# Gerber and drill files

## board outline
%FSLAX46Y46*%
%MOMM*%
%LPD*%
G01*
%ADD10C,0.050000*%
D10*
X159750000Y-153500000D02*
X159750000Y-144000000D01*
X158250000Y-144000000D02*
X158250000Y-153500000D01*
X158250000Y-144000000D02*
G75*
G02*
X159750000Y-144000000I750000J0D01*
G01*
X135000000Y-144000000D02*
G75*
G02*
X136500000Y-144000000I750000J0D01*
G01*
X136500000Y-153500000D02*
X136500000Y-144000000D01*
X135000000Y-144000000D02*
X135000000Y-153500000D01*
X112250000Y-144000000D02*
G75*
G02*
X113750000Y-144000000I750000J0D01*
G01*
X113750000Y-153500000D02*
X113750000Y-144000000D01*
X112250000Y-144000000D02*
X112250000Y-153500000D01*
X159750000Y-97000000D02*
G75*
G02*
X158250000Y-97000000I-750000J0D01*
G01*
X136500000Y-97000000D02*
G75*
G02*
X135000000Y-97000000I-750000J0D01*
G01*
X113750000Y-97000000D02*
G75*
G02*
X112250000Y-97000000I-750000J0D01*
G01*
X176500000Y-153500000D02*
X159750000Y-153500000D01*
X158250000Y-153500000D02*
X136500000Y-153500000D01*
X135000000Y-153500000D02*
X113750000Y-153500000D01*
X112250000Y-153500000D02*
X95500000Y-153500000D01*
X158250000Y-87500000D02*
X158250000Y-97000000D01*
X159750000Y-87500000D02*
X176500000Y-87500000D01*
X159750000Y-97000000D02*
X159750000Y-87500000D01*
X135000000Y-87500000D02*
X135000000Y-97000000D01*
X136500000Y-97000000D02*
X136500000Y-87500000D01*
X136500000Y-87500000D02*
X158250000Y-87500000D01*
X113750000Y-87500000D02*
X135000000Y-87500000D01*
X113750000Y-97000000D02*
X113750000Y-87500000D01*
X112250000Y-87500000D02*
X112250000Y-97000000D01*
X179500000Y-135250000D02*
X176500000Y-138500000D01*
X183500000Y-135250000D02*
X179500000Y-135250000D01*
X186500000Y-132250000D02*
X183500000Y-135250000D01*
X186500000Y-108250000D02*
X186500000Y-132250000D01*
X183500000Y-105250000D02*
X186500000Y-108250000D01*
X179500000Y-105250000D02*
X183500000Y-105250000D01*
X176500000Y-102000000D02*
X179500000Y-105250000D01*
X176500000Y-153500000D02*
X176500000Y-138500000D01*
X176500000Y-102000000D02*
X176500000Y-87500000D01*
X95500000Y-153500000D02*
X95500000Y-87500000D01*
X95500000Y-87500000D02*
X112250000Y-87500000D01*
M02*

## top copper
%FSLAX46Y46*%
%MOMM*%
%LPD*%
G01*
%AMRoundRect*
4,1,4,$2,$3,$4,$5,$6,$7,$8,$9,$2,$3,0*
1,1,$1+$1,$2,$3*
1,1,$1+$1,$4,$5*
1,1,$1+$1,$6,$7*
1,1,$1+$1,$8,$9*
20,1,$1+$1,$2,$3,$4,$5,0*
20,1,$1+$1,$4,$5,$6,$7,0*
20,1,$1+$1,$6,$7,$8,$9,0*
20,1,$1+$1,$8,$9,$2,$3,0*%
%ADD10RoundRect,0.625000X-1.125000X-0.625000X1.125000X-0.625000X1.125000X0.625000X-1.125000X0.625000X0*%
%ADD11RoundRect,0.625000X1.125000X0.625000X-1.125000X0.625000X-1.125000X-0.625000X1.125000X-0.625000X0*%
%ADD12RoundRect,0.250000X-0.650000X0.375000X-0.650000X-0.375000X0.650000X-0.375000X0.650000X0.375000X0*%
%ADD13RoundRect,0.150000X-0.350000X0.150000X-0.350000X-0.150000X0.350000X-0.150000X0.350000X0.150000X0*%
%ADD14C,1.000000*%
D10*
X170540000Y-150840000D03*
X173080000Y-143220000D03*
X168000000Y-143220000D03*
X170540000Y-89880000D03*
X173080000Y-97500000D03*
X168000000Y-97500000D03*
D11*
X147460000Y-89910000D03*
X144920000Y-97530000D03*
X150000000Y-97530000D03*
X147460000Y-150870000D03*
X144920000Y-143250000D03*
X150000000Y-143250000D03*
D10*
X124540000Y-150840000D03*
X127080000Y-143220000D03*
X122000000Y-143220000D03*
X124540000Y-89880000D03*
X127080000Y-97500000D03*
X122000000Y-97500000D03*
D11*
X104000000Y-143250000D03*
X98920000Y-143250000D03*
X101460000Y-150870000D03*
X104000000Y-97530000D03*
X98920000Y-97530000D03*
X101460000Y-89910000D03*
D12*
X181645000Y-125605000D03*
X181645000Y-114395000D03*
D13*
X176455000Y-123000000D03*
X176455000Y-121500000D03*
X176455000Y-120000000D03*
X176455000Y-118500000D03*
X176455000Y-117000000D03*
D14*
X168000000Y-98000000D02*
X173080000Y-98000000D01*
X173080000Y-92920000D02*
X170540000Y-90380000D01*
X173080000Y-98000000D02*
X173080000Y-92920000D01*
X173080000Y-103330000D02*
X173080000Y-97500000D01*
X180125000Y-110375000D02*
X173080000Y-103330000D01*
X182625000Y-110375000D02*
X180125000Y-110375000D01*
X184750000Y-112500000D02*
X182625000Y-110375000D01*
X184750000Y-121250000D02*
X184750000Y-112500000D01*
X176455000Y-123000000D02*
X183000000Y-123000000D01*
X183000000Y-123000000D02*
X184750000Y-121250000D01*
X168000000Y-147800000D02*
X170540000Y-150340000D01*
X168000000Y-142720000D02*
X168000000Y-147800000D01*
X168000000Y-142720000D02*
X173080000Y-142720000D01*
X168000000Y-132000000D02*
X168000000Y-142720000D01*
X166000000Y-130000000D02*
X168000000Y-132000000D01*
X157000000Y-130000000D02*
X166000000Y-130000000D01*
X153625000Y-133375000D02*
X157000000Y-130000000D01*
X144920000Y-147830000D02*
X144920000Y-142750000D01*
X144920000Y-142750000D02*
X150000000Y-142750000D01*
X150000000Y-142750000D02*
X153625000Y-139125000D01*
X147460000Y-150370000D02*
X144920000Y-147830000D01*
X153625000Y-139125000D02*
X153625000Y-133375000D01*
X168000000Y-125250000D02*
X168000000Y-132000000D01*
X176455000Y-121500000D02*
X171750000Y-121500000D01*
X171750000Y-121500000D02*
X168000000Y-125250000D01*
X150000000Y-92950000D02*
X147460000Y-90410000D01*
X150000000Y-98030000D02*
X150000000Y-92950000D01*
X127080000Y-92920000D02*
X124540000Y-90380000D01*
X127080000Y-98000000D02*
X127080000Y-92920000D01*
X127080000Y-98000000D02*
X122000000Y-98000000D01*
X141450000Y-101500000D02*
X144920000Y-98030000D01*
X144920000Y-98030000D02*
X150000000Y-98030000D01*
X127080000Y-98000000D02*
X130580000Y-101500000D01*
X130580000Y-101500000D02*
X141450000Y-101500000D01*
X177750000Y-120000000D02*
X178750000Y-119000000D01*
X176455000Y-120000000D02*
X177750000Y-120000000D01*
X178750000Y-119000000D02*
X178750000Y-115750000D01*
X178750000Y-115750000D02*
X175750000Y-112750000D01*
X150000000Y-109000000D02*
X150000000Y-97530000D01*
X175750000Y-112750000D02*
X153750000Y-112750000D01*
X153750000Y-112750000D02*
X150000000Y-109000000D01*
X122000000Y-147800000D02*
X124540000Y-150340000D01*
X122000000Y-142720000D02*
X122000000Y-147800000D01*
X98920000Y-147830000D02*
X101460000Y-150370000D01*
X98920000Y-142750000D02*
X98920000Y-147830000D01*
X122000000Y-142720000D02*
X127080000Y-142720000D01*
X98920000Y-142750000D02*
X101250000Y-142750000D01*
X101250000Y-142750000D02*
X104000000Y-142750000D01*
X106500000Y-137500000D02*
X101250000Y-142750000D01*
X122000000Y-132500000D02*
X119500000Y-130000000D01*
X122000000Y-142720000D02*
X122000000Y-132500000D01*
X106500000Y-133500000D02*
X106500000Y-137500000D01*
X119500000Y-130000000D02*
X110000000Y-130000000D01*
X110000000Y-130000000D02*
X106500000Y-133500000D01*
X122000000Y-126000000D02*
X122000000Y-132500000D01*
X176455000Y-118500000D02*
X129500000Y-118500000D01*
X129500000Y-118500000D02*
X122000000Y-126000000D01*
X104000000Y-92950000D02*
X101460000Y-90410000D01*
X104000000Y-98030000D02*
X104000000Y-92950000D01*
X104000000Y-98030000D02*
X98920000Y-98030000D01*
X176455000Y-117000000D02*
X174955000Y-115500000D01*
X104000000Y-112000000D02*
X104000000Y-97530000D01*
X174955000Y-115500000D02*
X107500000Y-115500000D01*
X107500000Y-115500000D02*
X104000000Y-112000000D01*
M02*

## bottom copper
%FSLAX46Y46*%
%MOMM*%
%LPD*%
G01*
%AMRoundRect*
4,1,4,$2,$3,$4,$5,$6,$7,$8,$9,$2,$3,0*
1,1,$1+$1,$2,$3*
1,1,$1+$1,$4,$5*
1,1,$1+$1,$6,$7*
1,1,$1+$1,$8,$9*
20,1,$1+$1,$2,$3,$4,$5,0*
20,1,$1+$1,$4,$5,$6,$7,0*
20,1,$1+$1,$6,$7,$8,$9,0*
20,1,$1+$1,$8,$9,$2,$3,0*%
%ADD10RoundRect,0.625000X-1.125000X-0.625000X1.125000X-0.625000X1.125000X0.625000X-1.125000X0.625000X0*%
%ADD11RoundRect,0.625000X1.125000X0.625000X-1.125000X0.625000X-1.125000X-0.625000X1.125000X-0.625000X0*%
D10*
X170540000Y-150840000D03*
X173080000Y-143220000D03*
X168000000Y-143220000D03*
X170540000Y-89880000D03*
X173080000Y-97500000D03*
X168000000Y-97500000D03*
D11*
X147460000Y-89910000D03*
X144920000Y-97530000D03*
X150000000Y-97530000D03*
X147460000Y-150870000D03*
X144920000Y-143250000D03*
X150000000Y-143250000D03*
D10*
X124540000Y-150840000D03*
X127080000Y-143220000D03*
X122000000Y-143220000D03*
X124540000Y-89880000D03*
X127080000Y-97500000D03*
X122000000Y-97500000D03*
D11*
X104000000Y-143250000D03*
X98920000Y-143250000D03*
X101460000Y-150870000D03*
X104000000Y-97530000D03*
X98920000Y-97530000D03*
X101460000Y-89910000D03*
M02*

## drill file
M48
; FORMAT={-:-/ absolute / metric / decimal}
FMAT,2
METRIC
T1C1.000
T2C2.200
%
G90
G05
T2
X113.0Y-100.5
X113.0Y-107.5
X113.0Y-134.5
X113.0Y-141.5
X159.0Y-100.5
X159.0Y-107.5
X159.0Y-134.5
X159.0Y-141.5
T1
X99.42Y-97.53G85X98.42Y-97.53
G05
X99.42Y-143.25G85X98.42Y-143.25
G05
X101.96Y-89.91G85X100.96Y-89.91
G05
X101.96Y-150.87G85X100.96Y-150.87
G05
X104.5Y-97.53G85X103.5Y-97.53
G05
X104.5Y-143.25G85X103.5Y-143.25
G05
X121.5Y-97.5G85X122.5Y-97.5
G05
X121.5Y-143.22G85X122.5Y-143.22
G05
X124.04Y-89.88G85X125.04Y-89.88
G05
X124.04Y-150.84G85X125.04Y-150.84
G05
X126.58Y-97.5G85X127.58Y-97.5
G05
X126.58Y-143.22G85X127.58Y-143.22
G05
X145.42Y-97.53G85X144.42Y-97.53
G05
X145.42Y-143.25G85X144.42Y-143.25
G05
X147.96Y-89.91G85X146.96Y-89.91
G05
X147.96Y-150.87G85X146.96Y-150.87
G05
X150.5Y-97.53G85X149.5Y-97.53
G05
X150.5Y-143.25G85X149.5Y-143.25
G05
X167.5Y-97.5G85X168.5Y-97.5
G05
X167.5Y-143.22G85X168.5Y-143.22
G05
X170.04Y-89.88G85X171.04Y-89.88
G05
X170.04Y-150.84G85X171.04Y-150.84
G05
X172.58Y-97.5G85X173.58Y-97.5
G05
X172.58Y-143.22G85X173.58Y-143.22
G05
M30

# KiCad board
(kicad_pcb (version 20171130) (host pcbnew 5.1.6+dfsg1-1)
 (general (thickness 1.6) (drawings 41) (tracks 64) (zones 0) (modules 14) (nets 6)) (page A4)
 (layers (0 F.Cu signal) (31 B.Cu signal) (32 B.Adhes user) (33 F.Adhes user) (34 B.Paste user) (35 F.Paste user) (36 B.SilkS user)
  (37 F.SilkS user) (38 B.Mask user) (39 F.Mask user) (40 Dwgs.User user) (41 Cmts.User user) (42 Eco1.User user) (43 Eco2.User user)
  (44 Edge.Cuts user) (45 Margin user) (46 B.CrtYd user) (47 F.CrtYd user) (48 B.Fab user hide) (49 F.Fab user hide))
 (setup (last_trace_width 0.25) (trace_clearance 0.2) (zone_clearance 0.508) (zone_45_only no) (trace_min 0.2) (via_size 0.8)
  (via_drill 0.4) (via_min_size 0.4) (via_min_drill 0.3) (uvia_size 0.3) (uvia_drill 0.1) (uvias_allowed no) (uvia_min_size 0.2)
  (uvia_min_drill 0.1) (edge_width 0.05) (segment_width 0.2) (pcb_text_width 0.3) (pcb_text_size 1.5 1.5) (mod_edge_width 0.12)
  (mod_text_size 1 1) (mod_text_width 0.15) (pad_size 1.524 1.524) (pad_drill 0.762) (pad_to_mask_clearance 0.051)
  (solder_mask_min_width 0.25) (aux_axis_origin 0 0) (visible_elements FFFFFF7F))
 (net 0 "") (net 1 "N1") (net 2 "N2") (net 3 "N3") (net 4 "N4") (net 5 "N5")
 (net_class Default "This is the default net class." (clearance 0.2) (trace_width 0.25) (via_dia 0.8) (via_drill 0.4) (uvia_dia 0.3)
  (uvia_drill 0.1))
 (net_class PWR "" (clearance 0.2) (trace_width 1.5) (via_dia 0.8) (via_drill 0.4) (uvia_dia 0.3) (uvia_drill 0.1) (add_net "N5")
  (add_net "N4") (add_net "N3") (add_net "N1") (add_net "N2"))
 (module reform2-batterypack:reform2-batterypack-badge (layer F.Cu) (at 136 120.5 90)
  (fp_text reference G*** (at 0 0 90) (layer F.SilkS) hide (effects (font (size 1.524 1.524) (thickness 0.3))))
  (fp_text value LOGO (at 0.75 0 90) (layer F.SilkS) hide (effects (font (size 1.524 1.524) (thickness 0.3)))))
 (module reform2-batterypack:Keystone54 (layer F.Cu) (at 168 98)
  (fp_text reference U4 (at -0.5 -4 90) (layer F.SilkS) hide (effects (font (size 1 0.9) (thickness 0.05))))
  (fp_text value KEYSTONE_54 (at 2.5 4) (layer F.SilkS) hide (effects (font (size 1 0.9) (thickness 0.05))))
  (pad 6 thru_hole roundrect (at 2.54 52.84) (size 3.5 2.5) (drill oval 2 1) (layers *.Cu *.Mask) (roundrect_rratio 0.25) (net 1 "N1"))
  (pad 5 thru_hole roundrect (at 5.08 45.22) (size 3.5 2.5) (drill oval 2 1) (layers *.Cu *.Mask) (roundrect_rratio 0.25) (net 1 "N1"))
  (pad 4 thru_hole roundrect (at 0 45.22) (size 3.5 2.5) (drill oval 2 1) (layers *.Cu *.Mask) (roundrect_rratio 0.25) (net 1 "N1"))
  (pad 3 thru_hole roundrect (at 2.54 -8.12) (size 3.5 2.5) (drill oval 2 1) (layers *.Cu *.Mask) (roundrect_rratio 0.25) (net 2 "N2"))
  (pad 2 thru_hole roundrect (at 5.08 -0.5) (size 3.5 2.5) (drill oval 2 1) (layers *.Cu *.Mask) (roundrect_rratio 0.25) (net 2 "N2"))
  (pad 1 thru_hole roundrect (at 0 -0.5) (size 3.5 2.5) (drill oval 2 1) (layers *.Cu *.Mask) (roundrect_rratio 0.25) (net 2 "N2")))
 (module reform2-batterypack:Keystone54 (layer F.Cu) (at 150 142.75 180)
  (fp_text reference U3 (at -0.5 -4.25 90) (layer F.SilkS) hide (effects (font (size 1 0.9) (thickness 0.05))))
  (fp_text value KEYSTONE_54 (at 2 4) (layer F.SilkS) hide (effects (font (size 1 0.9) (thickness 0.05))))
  (pad 6 thru_hole roundrect (at 2.54 52.84 180) (size 3.5 2.5) (drill oval 2 1) (layers *.Cu *.Mask) (roundrect_rratio 0.25) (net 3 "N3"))
  (pad 5 thru_hole roundrect (at 5.08 45.22 180) (size 3.5 2.5) (drill oval 2 1) (layers *.Cu *.Mask) (roundrect_rratio 0.25) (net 3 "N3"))
  (pad 4 thru_hole roundrect (at 0 45.22 180) (size 3.5 2.5) (drill oval 2 1) (layers *.Cu *.Mask) (roundrect_rratio 0.25) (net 3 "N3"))
  (pad 3 thru_hole roundrect (at 2.54 -8.12 180) (size 3.5 2.5) (drill oval 2 1) (layers *.Cu *.Mask) (roundrect_rratio 0.25) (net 1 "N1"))
  (pad 2 thru_hole roundrect (at 5.08 -0.5 180) (size 3.5 2.5) (drill oval 2 1) (layers *.Cu *.Mask) (roundrect_rratio 0.25) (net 1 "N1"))
  (pad 1 thru_hole roundrect (at 0 -0.5 180) (size 3.5 2.5) (drill oval 2 1) (layers *.Cu *.Mask) (roundrect_rratio 0.25) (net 1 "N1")))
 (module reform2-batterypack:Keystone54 (layer F.Cu) (at 122 98)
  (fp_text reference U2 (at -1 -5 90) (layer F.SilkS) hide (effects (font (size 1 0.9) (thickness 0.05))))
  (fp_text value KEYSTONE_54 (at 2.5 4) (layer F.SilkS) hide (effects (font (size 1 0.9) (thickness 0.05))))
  (pad 6 thru_hole roundrect (at 2.54 52.84) (size 3.5 2.5) (drill oval 2 1) (layers *.Cu *.Mask) (roundrect_rratio 0.25) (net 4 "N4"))
  (pad 5 thru_hole roundrect (at 5.08 45.22) (size 3.5 2.5) (drill oval 2 1) (layers *.Cu *.Mask) (roundrect_rratio 0.25) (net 4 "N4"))
  (pad 4 thru_hole roundrect (at 0 45.22) (size 3.5 2.5) (drill oval 2 1) (layers *.Cu *.Mask) (roundrect_rratio 0.25) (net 4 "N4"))
  (pad 3 thru_hole roundrect (at 2.54 -8.12) (size 3.5 2.5) (drill oval 2 1) (layers *.Cu *.Mask) (roundrect_rratio 0.25) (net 3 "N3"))
  (pad 2 thru_hole roundrect (at 5.08 -0.5) (size 3.5 2.5) (drill oval 2 1) (layers *.Cu *.Mask) (roundrect_rratio 0.25) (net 3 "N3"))
  (pad 1 thru_hole roundrect (at 0 -0.5) (size 3.5 2.5) (drill oval 2 1) (layers *.Cu *.Mask) (roundrect_rratio 0.25) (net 3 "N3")))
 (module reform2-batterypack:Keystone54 (layer F.Cu) (at 104 142.75 180)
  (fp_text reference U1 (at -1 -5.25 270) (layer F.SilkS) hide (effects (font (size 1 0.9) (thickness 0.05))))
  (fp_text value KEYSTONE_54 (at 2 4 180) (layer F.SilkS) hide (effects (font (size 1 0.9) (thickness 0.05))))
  (pad 1 thru_hole roundrect (at 0 -0.5 180) (size 3.5 2.5) (drill oval 2 1) (layers *.Cu *.Mask) (roundrect_rratio 0.25) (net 4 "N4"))
  (pad 2 thru_hole roundrect (at 5.08 -0.5 180) (size 3.5 2.5) (drill oval 2 1) (layers *.Cu *.Mask) (roundrect_rratio 0.25) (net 4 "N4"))
  (pad 3 thru_hole roundrect (at 2.54 -8.12 180) (size 3.5 2.5) (drill oval 2 1) (layers *.Cu *.Mask) (roundrect_rratio 0.25) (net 4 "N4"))
  (pad 4 thru_hole roundrect (at 0 45.22 180) (size 3.5 2.5) (drill oval 2 1) (layers *.Cu *.Mask) (roundrect_rratio 0.25) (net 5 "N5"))
  (pad 5 thru_hole roundrect (at 5.08 45.22 180) (size 3.5 2.5) (drill oval 2 1) (layers *.Cu *.Mask) (roundrect_rratio 0.25) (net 5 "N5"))
  (pad 6 thru_hole roundrect (at 2.54 52.84 180) (size 3.5 2.5) (drill oval 2 1) (layers *.Cu *.Mask) (roundrect_rratio 0.25) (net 5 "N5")))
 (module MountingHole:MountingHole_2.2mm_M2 (layer F.Cu) (at 159 141.5)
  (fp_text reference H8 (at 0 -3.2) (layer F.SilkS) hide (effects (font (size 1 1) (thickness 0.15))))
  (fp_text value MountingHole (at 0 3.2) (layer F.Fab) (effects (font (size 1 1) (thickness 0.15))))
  (pad 1 np_thru_hole circle (at 0 0) (size 2.2 2.2) (drill 2.2) (layers *.Cu *.Mask)))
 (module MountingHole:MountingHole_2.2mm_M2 (layer F.Cu) (at 113 141.5)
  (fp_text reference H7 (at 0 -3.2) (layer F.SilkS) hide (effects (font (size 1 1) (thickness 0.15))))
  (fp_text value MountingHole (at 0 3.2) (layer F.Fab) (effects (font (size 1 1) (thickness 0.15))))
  (pad 1 np_thru_hole circle (at 0 0) (size 2.2 2.2) (drill 2.2) (layers *.Cu *.Mask)))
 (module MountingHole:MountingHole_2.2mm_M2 (layer F.Cu) (at 159 107.5)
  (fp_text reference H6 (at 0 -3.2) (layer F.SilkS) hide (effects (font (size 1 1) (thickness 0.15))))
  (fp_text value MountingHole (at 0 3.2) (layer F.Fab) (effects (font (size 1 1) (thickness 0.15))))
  (pad 1 np_thru_hole circle (at 0 0) (size 2.2 2.2) (drill 2.2) (layers *.Cu *.Mask)))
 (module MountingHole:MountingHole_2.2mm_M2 (layer F.Cu) (at 113 107.5)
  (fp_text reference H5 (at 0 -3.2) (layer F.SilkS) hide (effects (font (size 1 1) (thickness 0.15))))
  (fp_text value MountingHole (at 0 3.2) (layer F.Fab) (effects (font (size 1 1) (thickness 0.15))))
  (pad 1 np_thru_hole circle (at 0 0) (size 2.2 2.2) (drill 2.2) (layers *.Cu *.Mask)))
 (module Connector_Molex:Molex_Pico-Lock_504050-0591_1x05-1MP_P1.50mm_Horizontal (layer F.Cu) (at 179.25 120 270)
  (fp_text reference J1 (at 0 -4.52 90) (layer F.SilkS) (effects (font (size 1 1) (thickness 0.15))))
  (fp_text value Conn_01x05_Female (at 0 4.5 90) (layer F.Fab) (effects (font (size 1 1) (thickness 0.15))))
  (pad MP smd roundrect (at 5.605 -2.395 270) (size 1.25 1.8) (layers F.Cu F.Paste F.Mask) (roundrect_rratio 0.2))
  (pad MP smd roundrect (at -5.605 -2.395 270) (size 1.25 1.8) (layers F.Cu F.Paste F.Mask) (roundrect_rratio 0.2))
  (pad 5 smd roundrect (at 3 2.795 270) (size 0.6 1) (layers F.Cu F.Paste F.Mask) (roundrect_rratio 0.25) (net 2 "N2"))
  (pad 4 smd roundrect (at 1.5 2.795 270) (size 0.6 1) (layers F.Cu F.Paste F.Mask) (roundrect_rratio 0.25) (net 1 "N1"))
  (pad 3 smd roundrect (at 0 2.795 270) (size 0.6 1) (layers F.Cu F.Paste F.Mask) (roundrect_rratio 0.25) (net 3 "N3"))
  (pad 2 smd roundrect (at -1.5 2.795 270) (size 0.6 1) (layers F.Cu F.Paste F.Mask) (roundrect_rratio 0.25) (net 4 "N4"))
  (pad 1 smd roundrect (at -3 2.795 270) (size 0.6 1) (layers F.Cu F.Paste F.Mask) (roundrect_rratio 0.25) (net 5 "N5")))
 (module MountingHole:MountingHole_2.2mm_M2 (layer F.Cu) (at 159 134.5)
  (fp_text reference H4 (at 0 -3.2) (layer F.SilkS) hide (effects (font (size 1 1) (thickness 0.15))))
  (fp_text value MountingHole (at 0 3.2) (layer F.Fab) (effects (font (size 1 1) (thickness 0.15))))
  (pad 1 np_thru_hole circle (at 0 0) (size 2.2 2.2) (drill 2.2) (layers *.Cu *.Mask)))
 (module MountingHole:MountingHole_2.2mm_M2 (layer F.Cu) (at 113 134.5)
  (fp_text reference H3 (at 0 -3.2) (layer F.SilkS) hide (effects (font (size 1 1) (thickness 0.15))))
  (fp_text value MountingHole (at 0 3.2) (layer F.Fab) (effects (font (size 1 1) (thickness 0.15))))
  (pad 1 np_thru_hole circle (at 0 0) (size 2.2 2.2) (drill 2.2) (layers *.Cu *.Mask)))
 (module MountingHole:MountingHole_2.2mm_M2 (layer F.Cu) (at 159 100.5)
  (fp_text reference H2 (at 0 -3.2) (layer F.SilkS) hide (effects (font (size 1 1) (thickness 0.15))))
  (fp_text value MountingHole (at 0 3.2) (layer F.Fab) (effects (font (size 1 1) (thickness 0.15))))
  (pad 1 np_thru_hole circle (at 0 0) (size 2.2 2.2) (drill 2.2) (layers *.Cu *.Mask)))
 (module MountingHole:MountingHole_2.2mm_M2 (layer F.Cu) (at 113 100.5)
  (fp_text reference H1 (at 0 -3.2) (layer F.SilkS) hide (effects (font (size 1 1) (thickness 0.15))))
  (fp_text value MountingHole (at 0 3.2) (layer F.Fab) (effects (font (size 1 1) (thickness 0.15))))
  (pad 1 np_thru_hole circle (at 0 0) (size 2.2 2.2) (drill 2.2) (layers *.Cu *.Mask)))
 (gr_line (start 159.75 153.5) (end 159.75 144) (layer Edge.Cuts) (width 0.05))
 (gr_line (start 158.25 144) (end 158.25 153.5) (layer Edge.Cuts) (width 0.05))
 (gr_arc (start 159 144) (end 159.75 144) (angle -180) (layer Edge.Cuts) (width 0.05))
 (gr_arc (start 135.75 144) (end 136.5 144) (angle -180) (layer Edge.Cuts) (width 0.05))
 (gr_line (start 136.5 153.5) (end 136.5 144) (layer Edge.Cuts) (width 0.05))
 (gr_line (start 135 144) (end 135 153.5) (layer Edge.Cuts) (width 0.05))
 (gr_arc (start 113 144) (end 113.75 144) (angle -180) (layer Edge.Cuts) (width 0.05))
 (gr_line (start 113.75 153.5) (end 113.75 144) (layer Edge.Cuts) (width 0.05))
 (gr_line (start 112.25 144) (end 112.25 153.5) (layer Edge.Cuts) (width 0.05))
 (gr_arc (start 159 97) (end 158.25 97) (angle -180) (layer Edge.Cuts) (width 0.05))
 (gr_arc (start 135.75 97) (end 135 97) (angle -180) (layer Edge.Cuts) (width 0.05))
 (gr_arc (start 113 97) (end 112.25 97) (angle -180) (layer Edge.Cuts) (width 0.05))
 (gr_line (start 176.5 153.5) (end 159.75 153.5) (layer Edge.Cuts) (width 0.05))
 (gr_line (start 158.25 153.5) (end 136.5 153.5) (layer Edge.Cuts) (width 0.05))
 (gr_line (start 135 153.5) (end 113.75 153.5) (layer Edge.Cuts) (width 0.05))
 (gr_line (start 112.25 153.5) (end 95.5 153.5) (layer Edge.Cuts) (width 0.05))
 (gr_line (start 158.25 87.5) (end 158.25 97) (layer Edge.Cuts) (width 0.05))
 (gr_line (start 159.75 87.5) (end 176.5 87.5) (layer Edge.Cuts) (width 0.05))
 (gr_line (start 159.75 97) (end 159.75 87.5) (layer Edge.Cuts) (width 0.05))
 (gr_line (start 135 87.5) (end 135 97) (layer Edge.Cuts) (width 0.05))
 (gr_line (start 136.5 97) (end 136.5 87.5) (layer Edge.Cuts) (width 0.05))
 (gr_line (start 136.5 87.5) (end 158.25 87.5) (layer Edge.Cuts) (width 0.05))
 (gr_line (start 113.75 87.5) (end 135 87.5) (layer Edge.Cuts) (width 0.05))
 (gr_line (start 113.75 97) (end 113.75 87.5) (layer Edge.Cuts) (width 0.05))
 (gr_line (start 112.25 87.5) (end 112.25 97) (layer Edge.Cuts) (width 0.05))
 (gr_line (start 179.5 135.25) (end 176.5 138.5) (layer Edge.Cuts) (width 0.05))
 (gr_line (start 183.5 135.25) (end 179.5 135.25) (layer Edge.Cuts) (width 0.05))
 (gr_line (start 186.5 132.25) (end 183.5 135.25) (layer Edge.Cuts) (width 0.05))
 (gr_line (start 186.5 108.25) (end 186.5 132.25) (layer Edge.Cuts) (width 0.05))
 (gr_line (start 183.5 105.25) (end 186.5 108.25) (layer Edge.Cuts) (width 0.05))
 (gr_line (start 179.5 105.25) (end 183.5 105.25) (layer Edge.Cuts) (width 0.05))
 (gr_line (start 176.5 102) (end 179.5 105.25) (layer Edge.Cuts) (width 0.05))
 (gr_line (start 176.5 153.5) (end 176.5 138.5) (layer Edge.Cuts) (width 0.05))
 (gr_line (start 176.5 102) (end 176.5 87.5) (layer Edge.Cuts) (width 0.05))
 (gr_line (start 95.5 153.5) (end 95.5 87.5) (layer Edge.Cuts) (width 0.05))
 (gr_line (start 95.5 87.5) (end 112.25 87.5) (layer Edge.Cuts) (width 0.05))
 (segment (start 168 98) (end 173.08 98) (width 1) (layer F.Cu) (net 2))
 (segment (start 173.08 92.92) (end 170.54 90.38) (width 1) (layer F.Cu) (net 2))
 (segment (start 173.08 98) (end 173.08 92.92) (width 1) (layer F.Cu) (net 2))
 (segment (start 173.08 103.33) (end 173.08 97.5) (width 1) (layer F.Cu) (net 2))
 (segment (start 180.125 110.375) (end 173.08 103.33) (width 1) (layer F.Cu) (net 2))
 (segment (start 182.625 110.375) (end 180.125 110.375) (width 1) (layer F.Cu) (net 2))
 (segment (start 184.75 112.5) (end 182.625 110.375) (width 1) (layer F.Cu) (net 2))
 (segment (start 184.75 121.25) (end 184.75 112.5) (width 1) (layer F.Cu) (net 2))
 (segment (start 176.455 123) (end 183 123) (width 1) (layer F.Cu) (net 2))
 (segment (start 183 123) (end 184.75 121.25) (width 1) (layer F.Cu) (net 2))
 (segment (start 168 147.8) (end 170.54 150.34) (width 1) (layer F.Cu) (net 1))
 (segment (start 168 142.72) (end 168 147.8) (width 1) (layer F.Cu) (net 1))
 (segment (start 168 142.72) (end 173.08 142.72) (width 1) (layer F.Cu) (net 1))
 (segment (start 168 132) (end 168 142.72) (width 1) (layer F.Cu) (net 1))
 (segment (start 166 130) (end 168 132) (width 1) (layer F.Cu) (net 1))
 (segment (start 157 130) (end 166 130) (width 1) (layer F.Cu) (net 1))
 (segment (start 153.625 133.375) (end 157 130) (width 1) (layer F.Cu) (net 1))
 (segment (start 144.92 147.83) (end 144.92 142.75) (width 1) (layer F.Cu) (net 1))
 (segment (start 144.92 142.75) (end 150 142.75) (width 1) (layer F.Cu) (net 1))
 (segment (start 150 142.75) (end 153.625 139.125) (width 1) (layer F.Cu) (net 1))
 (segment (start 147.46 150.37) (end 144.92 147.83) (width 1) (layer F.Cu) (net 1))
 (segment (start 153.625 139.125) (end 153.625 133.375) (width 1) (layer F.Cu) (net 1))
 (segment (start 168 125.25) (end 168 132) (width 1) (layer F.Cu) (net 1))
 (segment (start 176.455 121.5) (end 171.75 121.5) (width 1) (layer F.Cu) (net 1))
 (segment (start 171.75 121.5) (end 168 125.25) (width 1) (layer F.Cu) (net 1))
 (segment (start 150 92.95) (end 147.46 90.41) (width 1) (layer F.Cu) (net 3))
 (segment (start 150 98.03) (end 150 92.95) (width 1) (layer F.Cu) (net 3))
 (segment (start 127.08 92.92) (end 124.54 90.38) (width 1) (layer F.Cu) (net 3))
 (segment (start 127.08 98) (end 127.08 92.92) (width 1) (layer F.Cu) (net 3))
 (segment (start 127.08 98) (end 122 98) (width 1) (layer F.Cu) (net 3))
 (segment (start 141.45 101.5) (end 144.92 98.03) (width 1) (layer F.Cu) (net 3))
 (segment (start 144.92 98.03) (end 150 98.03) (width 1) (layer F.Cu) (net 3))
 (segment (start 127.08 98) (end 130.58 101.5) (width 1) (layer F.Cu) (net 3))
 (segment (start 130.58 101.5) (end 141.45 101.5) (width 1) (layer F.Cu) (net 3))
 (segment (start 177.75 120) (end 178.75 119) (width 1) (layer F.Cu) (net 3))
 (segment (start 176.455 120) (end 177.75 120) (width 1) (layer F.Cu) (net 3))
 (segment (start 178.75 119) (end 178.75 115.75) (width 1) (layer F.Cu) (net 3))
 (segment (start 178.75 115.75) (end 175.75 112.75) (width 1) (layer F.Cu) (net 3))
 (segment (start 150 109) (end 150 97.53) (width 1) (layer F.Cu) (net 3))
 (segment (start 175.75 112.75) (end 153.75 112.75) (width 1) (layer F.Cu) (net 3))
 (segment (start 153.75 112.75) (end 150 109) (width 1) (layer F.Cu) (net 3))
 (segment (start 122 147.8) (end 124.54 150.34) (width 1) (layer F.Cu) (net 4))
 (segment (start 122 142.72) (end 122 147.8) (width 1) (layer F.Cu) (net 4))
 (segment (start 98.92 147.83) (end 101.46 150.37) (width 1) (layer F.Cu) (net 4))
 (segment (start 98.92 142.75) (end 98.92 147.83) (width 1) (layer F.Cu) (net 4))
 (segment (start 122 142.72) (end 127.08 142.72) (width 1) (layer F.Cu) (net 4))
 (segment (start 98.92 142.75) (end 101.25 142.75) (width 1) (layer F.Cu) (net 4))
 (segment (start 101.25 142.75) (end 104 142.75) (width 1) (layer F.Cu) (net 4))
 (segment (start 106.5 137.5) (end 101.25 142.75) (width 1) (layer F.Cu) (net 4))
 (segment (start 122 132.5) (end 119.5 130) (width 1) (layer F.Cu) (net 4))
 (segment (start 122 142.72) (end 122 132.5) (width 1) (layer F.Cu) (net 4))
 (segment (start 106.5 133.5) (end 106.5 137.5) (width 1) (layer F.Cu) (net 4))
 (segment (start 119.5 130) (end 110 130) (width 1) (layer F.Cu) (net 4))
 (segment (start 110 130) (end 106.5 133.5) (width 1) (layer F.Cu) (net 4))
 (segment (start 122 126) (end 122 132.5) (width 1) (layer F.Cu) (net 4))
 (segment (start 176.455 118.5) (end 129.5 118.5) (width 1) (layer F.Cu) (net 4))
 (segment (start 129.5 118.5) (end 122 126) (width 1) (layer F.Cu) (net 4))
 (segment (start 104 92.95) (end 101.46 90.41) (width 1) (layer F.Cu) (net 5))
 (segment (start 104 98.03) (end 104 92.95) (width 1) (layer F.Cu) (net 5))
 (segment (start 104 98.03) (end 98.92 98.03) (width 1) (layer F.Cu) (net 5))
 (segment (start 176.455 117) (end 174.955 115.5) (width 1) (layer F.Cu) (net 5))
 (segment (start 104 112) (end 104 97.53) (width 1) (layer F.Cu) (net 5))
 (segment (start 174.955 115.5) (end 107.5 115.5) (width 1) (layer F.Cu) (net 5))
 (segment (start 107.5 115.5) (end 104 112) (width 1) (layer F.Cu) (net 5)))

